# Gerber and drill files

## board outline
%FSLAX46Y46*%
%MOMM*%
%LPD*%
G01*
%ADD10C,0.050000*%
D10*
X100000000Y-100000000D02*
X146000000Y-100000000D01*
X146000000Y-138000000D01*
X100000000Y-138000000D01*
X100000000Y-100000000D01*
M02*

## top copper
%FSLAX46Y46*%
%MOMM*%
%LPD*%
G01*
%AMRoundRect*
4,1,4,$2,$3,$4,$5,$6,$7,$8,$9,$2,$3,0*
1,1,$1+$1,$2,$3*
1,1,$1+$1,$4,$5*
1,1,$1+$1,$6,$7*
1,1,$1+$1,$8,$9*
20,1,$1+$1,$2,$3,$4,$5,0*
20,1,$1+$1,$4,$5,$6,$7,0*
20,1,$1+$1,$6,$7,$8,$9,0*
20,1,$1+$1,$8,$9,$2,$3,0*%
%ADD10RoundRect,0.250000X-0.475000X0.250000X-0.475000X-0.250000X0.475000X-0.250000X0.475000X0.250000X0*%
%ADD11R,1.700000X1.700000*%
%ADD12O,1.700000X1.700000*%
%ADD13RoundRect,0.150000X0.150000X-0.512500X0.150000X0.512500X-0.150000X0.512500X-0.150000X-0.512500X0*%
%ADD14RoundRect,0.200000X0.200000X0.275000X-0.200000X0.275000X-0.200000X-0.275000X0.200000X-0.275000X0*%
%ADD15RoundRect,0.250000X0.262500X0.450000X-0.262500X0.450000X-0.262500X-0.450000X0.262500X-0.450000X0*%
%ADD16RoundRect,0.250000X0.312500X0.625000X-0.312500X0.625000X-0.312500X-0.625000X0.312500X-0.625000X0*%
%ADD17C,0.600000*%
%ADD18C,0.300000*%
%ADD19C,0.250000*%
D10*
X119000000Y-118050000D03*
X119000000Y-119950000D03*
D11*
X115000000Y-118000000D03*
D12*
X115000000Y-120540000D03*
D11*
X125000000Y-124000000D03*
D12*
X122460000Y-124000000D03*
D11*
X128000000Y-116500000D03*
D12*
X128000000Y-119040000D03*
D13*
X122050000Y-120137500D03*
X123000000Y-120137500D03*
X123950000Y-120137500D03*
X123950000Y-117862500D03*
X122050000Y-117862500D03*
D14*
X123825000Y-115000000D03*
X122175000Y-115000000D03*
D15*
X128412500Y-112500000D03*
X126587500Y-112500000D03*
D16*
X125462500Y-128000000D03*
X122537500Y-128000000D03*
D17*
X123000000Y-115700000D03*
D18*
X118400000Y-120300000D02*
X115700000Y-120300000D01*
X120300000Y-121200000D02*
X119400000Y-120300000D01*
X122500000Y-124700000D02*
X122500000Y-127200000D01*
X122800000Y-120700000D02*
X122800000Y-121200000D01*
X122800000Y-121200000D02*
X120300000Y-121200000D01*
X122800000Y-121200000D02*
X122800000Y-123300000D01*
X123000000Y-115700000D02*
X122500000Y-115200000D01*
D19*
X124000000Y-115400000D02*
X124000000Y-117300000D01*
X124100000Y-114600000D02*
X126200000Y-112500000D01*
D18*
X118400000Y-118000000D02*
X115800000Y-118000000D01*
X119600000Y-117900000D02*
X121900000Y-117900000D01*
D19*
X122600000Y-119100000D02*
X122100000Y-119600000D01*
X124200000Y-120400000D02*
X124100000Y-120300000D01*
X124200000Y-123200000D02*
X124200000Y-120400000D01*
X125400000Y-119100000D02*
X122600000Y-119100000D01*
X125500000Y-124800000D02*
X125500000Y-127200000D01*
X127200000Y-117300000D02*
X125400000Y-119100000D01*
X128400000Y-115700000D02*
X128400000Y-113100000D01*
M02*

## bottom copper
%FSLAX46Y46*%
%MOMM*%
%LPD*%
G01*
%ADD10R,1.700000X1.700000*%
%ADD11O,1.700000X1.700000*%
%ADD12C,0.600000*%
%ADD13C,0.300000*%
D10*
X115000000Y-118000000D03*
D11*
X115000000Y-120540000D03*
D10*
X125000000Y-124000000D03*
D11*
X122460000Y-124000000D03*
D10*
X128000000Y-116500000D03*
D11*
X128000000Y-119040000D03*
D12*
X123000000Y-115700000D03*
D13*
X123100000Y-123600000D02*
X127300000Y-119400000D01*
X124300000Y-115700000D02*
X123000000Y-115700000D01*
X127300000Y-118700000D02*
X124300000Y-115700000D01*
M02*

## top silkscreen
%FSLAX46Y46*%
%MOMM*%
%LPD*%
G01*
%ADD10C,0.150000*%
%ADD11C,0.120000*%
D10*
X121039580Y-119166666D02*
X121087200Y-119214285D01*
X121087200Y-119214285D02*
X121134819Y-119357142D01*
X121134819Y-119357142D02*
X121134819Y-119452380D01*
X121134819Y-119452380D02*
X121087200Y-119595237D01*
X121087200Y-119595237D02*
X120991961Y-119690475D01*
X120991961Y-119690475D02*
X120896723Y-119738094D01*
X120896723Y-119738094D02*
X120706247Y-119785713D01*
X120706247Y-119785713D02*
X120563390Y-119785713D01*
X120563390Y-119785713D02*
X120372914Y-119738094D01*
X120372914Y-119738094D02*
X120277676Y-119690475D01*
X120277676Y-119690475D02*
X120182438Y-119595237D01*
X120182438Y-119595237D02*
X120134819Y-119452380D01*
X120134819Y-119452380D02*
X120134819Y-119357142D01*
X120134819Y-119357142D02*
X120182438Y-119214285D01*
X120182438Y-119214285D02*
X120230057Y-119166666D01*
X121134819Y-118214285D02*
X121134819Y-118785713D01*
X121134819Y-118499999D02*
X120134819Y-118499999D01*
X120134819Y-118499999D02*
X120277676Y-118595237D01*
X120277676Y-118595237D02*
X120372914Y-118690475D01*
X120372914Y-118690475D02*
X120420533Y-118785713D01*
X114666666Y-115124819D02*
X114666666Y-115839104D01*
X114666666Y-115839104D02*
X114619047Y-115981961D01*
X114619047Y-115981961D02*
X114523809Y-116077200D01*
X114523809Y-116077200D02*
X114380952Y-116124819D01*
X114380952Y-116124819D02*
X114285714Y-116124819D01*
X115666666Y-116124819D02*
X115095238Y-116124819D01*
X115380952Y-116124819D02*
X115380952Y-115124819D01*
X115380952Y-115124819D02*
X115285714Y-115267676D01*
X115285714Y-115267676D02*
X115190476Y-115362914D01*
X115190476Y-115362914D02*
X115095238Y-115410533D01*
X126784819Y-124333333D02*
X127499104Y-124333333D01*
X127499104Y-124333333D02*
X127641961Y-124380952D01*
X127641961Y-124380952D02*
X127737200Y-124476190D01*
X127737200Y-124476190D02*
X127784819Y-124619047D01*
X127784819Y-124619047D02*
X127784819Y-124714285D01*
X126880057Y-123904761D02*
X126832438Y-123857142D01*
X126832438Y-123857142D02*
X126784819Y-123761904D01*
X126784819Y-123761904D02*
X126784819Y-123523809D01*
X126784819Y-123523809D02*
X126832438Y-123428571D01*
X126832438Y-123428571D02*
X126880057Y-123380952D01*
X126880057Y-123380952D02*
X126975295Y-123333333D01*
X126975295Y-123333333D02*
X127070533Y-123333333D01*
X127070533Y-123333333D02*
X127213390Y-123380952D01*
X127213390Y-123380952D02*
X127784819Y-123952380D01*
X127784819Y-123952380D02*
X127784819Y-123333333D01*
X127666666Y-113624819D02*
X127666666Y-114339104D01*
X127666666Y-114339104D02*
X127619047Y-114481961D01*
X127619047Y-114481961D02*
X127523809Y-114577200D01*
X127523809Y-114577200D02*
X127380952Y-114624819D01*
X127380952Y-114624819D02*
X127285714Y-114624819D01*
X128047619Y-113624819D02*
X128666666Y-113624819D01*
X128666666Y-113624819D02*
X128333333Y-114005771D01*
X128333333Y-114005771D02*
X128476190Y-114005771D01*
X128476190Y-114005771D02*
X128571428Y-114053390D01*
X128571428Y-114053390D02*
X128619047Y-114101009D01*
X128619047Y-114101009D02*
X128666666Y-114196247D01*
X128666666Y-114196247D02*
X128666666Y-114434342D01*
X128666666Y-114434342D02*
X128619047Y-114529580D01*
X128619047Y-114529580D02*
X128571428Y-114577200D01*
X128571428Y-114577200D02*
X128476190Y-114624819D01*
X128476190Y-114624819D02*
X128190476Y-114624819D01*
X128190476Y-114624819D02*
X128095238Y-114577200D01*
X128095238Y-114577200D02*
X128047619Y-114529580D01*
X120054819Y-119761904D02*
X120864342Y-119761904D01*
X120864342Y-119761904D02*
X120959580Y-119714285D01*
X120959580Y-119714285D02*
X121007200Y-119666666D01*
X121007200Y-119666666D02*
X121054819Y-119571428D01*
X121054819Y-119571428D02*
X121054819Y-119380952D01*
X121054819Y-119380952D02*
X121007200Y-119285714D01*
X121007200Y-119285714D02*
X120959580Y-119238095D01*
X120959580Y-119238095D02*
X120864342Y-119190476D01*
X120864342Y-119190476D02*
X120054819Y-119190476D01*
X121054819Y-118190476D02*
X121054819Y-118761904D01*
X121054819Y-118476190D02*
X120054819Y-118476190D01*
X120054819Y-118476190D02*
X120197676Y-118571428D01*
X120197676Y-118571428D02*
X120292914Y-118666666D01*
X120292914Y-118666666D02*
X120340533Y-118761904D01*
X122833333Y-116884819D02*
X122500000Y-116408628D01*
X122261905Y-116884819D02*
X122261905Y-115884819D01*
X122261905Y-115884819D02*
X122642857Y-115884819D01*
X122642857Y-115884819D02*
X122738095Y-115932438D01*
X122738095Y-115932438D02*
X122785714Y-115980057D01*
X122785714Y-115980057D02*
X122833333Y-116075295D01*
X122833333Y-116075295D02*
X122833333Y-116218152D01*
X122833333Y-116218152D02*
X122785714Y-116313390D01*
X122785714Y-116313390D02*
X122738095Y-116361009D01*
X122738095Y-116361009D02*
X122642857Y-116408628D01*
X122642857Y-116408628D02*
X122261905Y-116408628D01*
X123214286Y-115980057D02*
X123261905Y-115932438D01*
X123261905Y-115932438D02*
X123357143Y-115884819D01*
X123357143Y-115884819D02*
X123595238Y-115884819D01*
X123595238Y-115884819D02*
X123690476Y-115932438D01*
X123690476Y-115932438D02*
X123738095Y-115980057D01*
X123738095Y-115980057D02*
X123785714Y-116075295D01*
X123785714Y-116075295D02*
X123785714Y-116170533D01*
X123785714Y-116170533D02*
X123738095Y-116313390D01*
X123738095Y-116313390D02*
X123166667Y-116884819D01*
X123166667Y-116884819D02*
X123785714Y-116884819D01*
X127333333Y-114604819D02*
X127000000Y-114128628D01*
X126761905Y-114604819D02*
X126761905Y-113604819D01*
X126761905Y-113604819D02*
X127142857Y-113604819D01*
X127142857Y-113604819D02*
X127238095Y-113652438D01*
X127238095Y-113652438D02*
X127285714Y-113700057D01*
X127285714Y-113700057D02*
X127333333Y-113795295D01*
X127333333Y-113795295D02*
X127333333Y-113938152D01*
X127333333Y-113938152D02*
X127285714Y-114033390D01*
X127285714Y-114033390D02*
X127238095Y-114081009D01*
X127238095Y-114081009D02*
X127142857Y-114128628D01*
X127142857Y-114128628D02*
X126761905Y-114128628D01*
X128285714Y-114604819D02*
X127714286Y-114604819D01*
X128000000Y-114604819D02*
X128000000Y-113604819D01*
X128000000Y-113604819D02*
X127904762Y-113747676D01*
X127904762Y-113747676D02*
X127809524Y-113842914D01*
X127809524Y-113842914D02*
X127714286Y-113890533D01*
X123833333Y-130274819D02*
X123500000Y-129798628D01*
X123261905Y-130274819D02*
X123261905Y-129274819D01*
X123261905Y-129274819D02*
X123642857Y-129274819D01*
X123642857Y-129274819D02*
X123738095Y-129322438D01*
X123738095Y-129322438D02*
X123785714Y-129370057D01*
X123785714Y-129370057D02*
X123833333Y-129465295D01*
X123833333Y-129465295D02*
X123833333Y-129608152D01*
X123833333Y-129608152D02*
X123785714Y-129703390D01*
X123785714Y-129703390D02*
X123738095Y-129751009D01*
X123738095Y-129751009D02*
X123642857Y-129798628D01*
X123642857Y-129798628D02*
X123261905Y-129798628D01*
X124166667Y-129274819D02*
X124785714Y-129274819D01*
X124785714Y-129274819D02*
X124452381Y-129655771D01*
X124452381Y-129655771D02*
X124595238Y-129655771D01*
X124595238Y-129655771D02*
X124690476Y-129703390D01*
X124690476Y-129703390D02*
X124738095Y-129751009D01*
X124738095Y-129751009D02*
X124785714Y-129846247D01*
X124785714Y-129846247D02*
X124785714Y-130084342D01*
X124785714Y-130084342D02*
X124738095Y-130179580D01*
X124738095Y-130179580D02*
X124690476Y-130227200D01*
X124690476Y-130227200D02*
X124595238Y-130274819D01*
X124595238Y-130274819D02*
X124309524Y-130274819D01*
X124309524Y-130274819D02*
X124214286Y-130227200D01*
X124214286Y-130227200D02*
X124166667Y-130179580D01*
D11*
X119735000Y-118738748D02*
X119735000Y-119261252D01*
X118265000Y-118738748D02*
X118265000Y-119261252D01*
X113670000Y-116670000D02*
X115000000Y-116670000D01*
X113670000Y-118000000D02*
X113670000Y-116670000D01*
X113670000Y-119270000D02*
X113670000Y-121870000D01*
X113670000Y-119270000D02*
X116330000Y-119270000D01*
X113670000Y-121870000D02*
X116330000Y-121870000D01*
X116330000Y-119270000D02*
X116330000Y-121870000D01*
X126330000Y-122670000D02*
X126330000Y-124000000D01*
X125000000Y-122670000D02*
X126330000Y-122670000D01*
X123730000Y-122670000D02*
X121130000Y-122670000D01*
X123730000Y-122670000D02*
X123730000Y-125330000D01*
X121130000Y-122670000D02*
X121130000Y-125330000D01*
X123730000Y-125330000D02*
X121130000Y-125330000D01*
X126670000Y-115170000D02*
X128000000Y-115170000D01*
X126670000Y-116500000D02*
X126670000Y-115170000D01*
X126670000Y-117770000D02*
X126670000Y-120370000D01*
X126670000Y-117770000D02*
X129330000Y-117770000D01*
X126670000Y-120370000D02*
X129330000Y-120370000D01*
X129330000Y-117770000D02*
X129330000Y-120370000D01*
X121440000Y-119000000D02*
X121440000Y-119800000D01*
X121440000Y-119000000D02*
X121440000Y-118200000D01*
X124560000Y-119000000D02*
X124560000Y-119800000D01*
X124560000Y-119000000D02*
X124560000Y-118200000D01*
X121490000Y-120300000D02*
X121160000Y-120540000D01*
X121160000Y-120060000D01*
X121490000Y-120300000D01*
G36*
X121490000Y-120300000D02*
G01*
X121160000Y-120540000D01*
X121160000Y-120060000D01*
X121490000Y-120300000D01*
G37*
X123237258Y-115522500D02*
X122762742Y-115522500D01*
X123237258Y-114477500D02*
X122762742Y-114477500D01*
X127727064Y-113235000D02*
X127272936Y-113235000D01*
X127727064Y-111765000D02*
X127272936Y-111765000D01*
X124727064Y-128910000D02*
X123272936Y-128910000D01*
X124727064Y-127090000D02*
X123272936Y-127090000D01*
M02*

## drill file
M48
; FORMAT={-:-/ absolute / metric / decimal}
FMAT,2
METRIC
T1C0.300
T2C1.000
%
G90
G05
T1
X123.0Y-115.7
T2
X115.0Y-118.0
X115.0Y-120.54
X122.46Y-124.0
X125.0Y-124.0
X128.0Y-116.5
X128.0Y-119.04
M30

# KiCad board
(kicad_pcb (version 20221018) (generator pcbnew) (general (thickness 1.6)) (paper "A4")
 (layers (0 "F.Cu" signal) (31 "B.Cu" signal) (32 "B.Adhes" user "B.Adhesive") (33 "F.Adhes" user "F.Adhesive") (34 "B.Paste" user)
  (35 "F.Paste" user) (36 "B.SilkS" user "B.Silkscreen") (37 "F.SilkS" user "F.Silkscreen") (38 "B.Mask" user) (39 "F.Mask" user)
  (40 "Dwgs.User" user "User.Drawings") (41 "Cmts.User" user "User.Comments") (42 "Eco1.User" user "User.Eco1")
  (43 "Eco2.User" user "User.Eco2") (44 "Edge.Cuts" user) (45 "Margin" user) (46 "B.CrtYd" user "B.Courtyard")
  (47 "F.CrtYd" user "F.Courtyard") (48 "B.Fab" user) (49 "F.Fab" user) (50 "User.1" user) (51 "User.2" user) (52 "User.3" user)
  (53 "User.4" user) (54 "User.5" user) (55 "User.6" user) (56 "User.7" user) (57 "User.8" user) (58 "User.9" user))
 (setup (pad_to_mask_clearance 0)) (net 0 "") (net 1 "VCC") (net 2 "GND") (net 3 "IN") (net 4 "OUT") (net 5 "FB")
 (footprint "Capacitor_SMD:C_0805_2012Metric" (layer "F.Cu") (at 119 119 -90)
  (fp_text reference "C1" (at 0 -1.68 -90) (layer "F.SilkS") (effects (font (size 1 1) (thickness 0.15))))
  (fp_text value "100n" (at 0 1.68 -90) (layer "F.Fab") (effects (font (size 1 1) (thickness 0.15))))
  (fp_line (start -0.261252 -0.735) (end 0.261252 -0.735) (stroke (width 0.12) (type solid)) (layer "F.SilkS"))
  (fp_line (start -0.261252 0.735) (end 0.261252 0.735) (stroke (width 0.12) (type solid)) (layer "F.SilkS"))
  (pad "1" smd roundrect (at -0.95 0 270) (size 1 1.45) (layers "F.Cu" "F.Paste" "F.Mask") (roundrect_rratio 0.25) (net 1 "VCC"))
  (pad "2" smd roundrect (at 0.95 0 270) (size 1 1.45) (layers "F.Cu" "F.Paste" "F.Mask") (roundrect_rratio 0.25) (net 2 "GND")))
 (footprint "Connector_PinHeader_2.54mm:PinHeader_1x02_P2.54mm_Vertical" (layer "F.Cu") (at 115 118)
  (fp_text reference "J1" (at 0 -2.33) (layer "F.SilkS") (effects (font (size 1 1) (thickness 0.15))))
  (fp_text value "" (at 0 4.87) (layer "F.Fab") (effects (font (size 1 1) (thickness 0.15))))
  (fp_line (start -1.33 -1.33) (end 0 -1.33) (stroke (width 0.12) (type solid)) (layer "F.SilkS"))
  (fp_line (start -1.33 0) (end -1.33 -1.33) (stroke (width 0.12) (type solid)) (layer "F.SilkS"))
  (fp_line (start -1.33 1.27) (end -1.33 3.87) (stroke (width 0.12) (type solid)) (layer "F.SilkS"))
  (fp_line (start -1.33 1.27) (end 1.33 1.27) (stroke (width 0.12) (type solid)) (layer "F.SilkS"))
  (fp_line (start -1.33 3.87) (end 1.33 3.87) (stroke (width 0.12) (type solid)) (layer "F.SilkS"))
  (fp_line (start 1.33 1.27) (end 1.33 3.87) (stroke (width 0.12) (type solid)) (layer "F.SilkS"))
  (pad "1" thru_hole rect (at 0 0) (size 1.7 1.7) (drill 1) (layers "*.Cu" "*.Mask") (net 1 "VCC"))
  (pad "2" thru_hole oval (at 0 2.54) (size 1.7 1.7) (drill 1) (layers "*.Cu" "*.Mask") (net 2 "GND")))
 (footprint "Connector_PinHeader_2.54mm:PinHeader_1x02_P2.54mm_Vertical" (layer "F.Cu") (at 125 124 -90)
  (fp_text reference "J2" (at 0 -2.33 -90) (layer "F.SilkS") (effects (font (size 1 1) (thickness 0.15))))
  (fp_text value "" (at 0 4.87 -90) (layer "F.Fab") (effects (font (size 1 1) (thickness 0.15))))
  (fp_line (start -1.33 -1.33) (end 0 -1.33) (stroke (width 0.12) (type solid)) (layer "F.SilkS"))
  (fp_line (start -1.33 0) (end -1.33 -1.33) (stroke (width 0.12) (type solid)) (layer "F.SilkS"))
  (fp_line (start -1.33 1.27) (end -1.33 3.87) (stroke (width 0.12) (type solid)) (layer "F.SilkS"))
  (fp_line (start -1.33 1.27) (end 1.33 1.27) (stroke (width 0.12) (type solid)) (layer "F.SilkS"))
  (fp_line (start -1.33 3.87) (end 1.33 3.87) (stroke (width 0.12) (type solid)) (layer "F.SilkS"))
  (fp_line (start 1.33 1.27) (end 1.33 3.87) (stroke (width 0.12) (type solid)) (layer "F.SilkS"))
  (pad "1" thru_hole rect (at 0 0 270) (size 1.7 1.7) (drill 1) (layers "*.Cu" "*.Mask") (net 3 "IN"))
  (pad "2" thru_hole oval (at 0 2.54 270) (size 1.7 1.7) (drill 1) (layers "*.Cu" "*.Mask") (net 2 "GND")))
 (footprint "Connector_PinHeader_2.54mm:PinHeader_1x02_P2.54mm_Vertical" (layer "F.Cu") (at 128 116.5)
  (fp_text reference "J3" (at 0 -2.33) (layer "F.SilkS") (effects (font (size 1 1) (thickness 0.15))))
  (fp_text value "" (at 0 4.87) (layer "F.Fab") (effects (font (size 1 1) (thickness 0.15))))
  (fp_line (start -1.33 -1.33) (end 0 -1.33) (stroke (width 0.12) (type solid)) (layer "F.SilkS"))
  (fp_line (start -1.33 0) (end -1.33 -1.33) (stroke (width 0.12) (type solid)) (layer "F.SilkS"))
  (fp_line (start -1.33 1.27) (end -1.33 3.87) (stroke (width 0.12) (type solid)) (layer "F.SilkS"))
  (fp_line (start -1.33 1.27) (end 1.33 1.27) (stroke (width 0.12) (type solid)) (layer "F.SilkS"))
  (fp_line (start -1.33 3.87) (end 1.33 3.87) (stroke (width 0.12) (type solid)) (layer "F.SilkS"))
  (fp_line (start 1.33 1.27) (end 1.33 3.87) (stroke (width 0.12) (type solid)) (layer "F.SilkS"))
  (pad "1" thru_hole rect (at 0 0) (size 1.7 1.7) (drill 1) (layers "*.Cu" "*.Mask") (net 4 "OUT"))
  (pad "2" thru_hole oval (at 0 2.54) (size 1.7 1.7) (drill 1) (layers "*.Cu" "*.Mask") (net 2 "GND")))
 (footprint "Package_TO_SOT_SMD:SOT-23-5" (layer "F.Cu") (at 123 119 90)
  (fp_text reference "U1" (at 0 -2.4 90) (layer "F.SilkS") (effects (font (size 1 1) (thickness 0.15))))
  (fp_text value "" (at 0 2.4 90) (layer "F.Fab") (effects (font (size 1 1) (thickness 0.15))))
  (fp_line (start 0 -1.56) (end -0.8 -1.56) (stroke (width 0.12) (type solid)) (layer "F.SilkS"))
  (fp_line (start 0 -1.56) (end 0.8 -1.56) (stroke (width 0.12) (type solid)) (layer "F.SilkS"))
  (fp_line (start 0 1.56) (end -0.8 1.56) (stroke (width 0.12) (type solid)) (layer "F.SilkS"))
  (fp_line (start 0 1.56) (end 0.8 1.56) (stroke (width 0.12) (type solid)) (layer "F.SilkS"))
  (fp_poly
   (pts (xy -1.3 -1.51) (xy -1.54 -1.84) (xy -1.06 -1.84) (xy -1.3 -1.51)) (stroke (width 0.12) (type solid)) (fill solid) (layer "F.SilkS"))
  (pad "1" smd roundrect (at -1.1375 -0.95 90) (size 1.325 0.6) (layers "F.Cu" "F.Paste" "F.Mask") (roundrect_rratio 0.25) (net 4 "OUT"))
  (pad "2" smd roundrect (at -1.1375 0 90) (size 1.325 0.6) (layers "F.Cu" "F.Paste" "F.Mask") (roundrect_rratio 0.25) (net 2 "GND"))
  (pad "3" smd roundrect (at -1.1375 0.95 90) (size 1.325 0.6) (layers "F.Cu" "F.Paste" "F.Mask") (roundrect_rratio 0.25) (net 3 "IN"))
  (pad "4" smd roundrect (at 1.1375 0.95 90) (size 1.325 0.6) (layers "F.Cu" "F.Paste" "F.Mask") (roundrect_rratio 0.25) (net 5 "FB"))
  (pad "5" smd roundrect (at 1.1375 -0.95 90) (size 1.325 0.6) (layers "F.Cu" "F.Paste" "F.Mask") (roundrect_rratio 0.25) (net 1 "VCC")))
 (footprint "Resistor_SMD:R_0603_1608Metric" (layer "F.Cu") (at 123 115 180)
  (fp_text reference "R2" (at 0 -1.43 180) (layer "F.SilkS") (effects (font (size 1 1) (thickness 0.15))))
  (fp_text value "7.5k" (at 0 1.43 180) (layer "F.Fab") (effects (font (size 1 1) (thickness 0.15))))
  (fp_line (start -0.237258 -0.5225) (end 0.237258 -0.5225) (stroke (width 0.12) (type solid)) (layer "F.SilkS"))
  (fp_line (start -0.237258 0.5225) (end 0.237258 0.5225) (stroke (width 0.12) (type solid)) (layer "F.SilkS"))
  (pad "1" smd roundrect (at -0.825 0 180) (size 0.8 0.95) (layers "F.Cu" "F.Paste" "F.Mask") (roundrect_rratio 0.25) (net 5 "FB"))
  (pad "2" smd roundrect (at 0.825 0 180) (size 0.8 0.95) (layers "F.Cu" "F.Paste" "F.Mask") (roundrect_rratio 0.25) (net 2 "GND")))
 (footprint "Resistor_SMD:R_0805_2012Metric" (layer "F.Cu") (at 127.5 112.5 180)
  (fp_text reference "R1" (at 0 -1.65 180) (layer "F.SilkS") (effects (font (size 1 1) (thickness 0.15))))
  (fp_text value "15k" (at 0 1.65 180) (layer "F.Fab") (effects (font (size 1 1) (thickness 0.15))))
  (fp_line (start -0.227064 -0.735) (end 0.227064 -0.735) (stroke (width 0.12) (type solid)) (layer "F.SilkS"))
  (fp_line (start -0.227064 0.735) (end 0.227064 0.735) (stroke (width 0.12) (type solid)) (layer "F.SilkS"))
  (pad "1" smd roundrect (at -0.9125 0 180) (size 1.025 1.4) (layers "F.Cu" "F.Paste" "F.Mask") (roundrect_rratio 0.243902) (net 4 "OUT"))
  (pad "2" smd roundrect (at 0.9125 0 180) (size 1.025 1.4) (layers "F.Cu" "F.Paste" "F.Mask") (roundrect_rratio 0.243902) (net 5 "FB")))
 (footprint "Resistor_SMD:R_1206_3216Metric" (layer "F.Cu") (at 124 128 180)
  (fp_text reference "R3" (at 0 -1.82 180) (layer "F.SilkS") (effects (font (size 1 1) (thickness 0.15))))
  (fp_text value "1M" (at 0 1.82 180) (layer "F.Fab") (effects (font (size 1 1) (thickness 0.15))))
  (fp_line (start -0.727064 -0.91) (end 0.727064 -0.91) (stroke (width 0.12) (type solid)) (layer "F.SilkS"))
  (fp_line (start -0.727064 0.91) (end 0.727064 0.91) (stroke (width 0.12) (type solid)) (layer "F.SilkS"))
  (pad "1" smd roundrect (at -1.4625 0 180) (size 1.125 1.75) (layers "F.Cu" "F.Paste" "F.Mask") (roundrect_rratio 0.222222) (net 3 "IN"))
  (pad "2" smd roundrect (at 1.4625 0 180) (size 1.125 1.75) (layers "F.Cu" "F.Paste" "F.Mask") (roundrect_rratio 0.222222) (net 2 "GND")))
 (gr_rect (start 100 100) (end 146 138) (stroke (width 0.05) (type default)) (fill none) (layer "Edge.Cuts"))
 (segment (start 118.4 120.3) (end 115.7 120.3) (width 0.3) (layer "F.Cu") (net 2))
 (segment (start 120.3 121.2) (end 119.4 120.3) (width 0.3) (layer "F.Cu") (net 2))
 (segment (start 122.5 124.7) (end 122.5 127.2) (width 0.3) (layer "F.Cu") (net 2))
 (segment (start 122.8 120.7) (end 122.8 121.2) (width 0.3) (layer "F.Cu") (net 2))
 (segment (start 122.8 121.2) (end 120.3 121.2) (width 0.3) (layer "F.Cu") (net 2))
 (segment (start 122.8 121.2) (end 122.8 123.3) (width 0.3) (layer "F.Cu") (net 2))
 (segment (start 123 115.7) (end 122.5 115.2) (width 0.3) (layer "F.Cu") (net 2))
 (segment (start 124 115.4) (end 124 117.3) (width 0.25) (layer "F.Cu") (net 5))
 (segment (start 124.1 114.6) (end 126.2 112.5) (width 0.25) (layer "F.Cu") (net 5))
 (via (at 123 115.7) (size 0.6) (drill 0.3) (layers "F.Cu" "B.Cu") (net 2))
 (segment (start 118.4 118) (end 115.8 118) (width 0.3) (layer "F.Cu") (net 1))
 (segment (start 119.6 117.9) (end 121.9 117.9) (width 0.3) (layer "F.Cu") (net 1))
 (segment (start 122.6 119.1) (end 122.1 119.6) (width 0.25) (layer "F.Cu") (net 4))
 (segment (start 123.1 123.6) (end 127.3 119.4) (width 0.3) (layer "B.Cu") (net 2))
 (segment (start 124.2 120.4) (end 124.1 120.3) (width 0.25) (layer "F.Cu") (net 3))
 (segment (start 124.2 123.2) (end 124.2 120.4) (width 0.25) (layer "F.Cu") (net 3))
 (segment (start 124.3 115.7) (end 123 115.7) (width 0.3) (layer "B.Cu") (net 2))
 (segment (start 125.4 119.1) (end 122.6 119.1) (width 0.25) (layer "F.Cu") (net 4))
 (segment (start 125.5 124.8) (end 125.5 127.2) (width 0.25) (layer "F.Cu") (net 3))
 (segment (start 127.2 117.3) (end 125.4 119.1) (width 0.25) (layer "F.Cu") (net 4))
 (segment (start 127.3 118.7) (end 124.3 115.7) (width 0.3) (layer "B.Cu") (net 2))
 (segment (start 128.4 115.7) (end 128.4 113.1) (width 0.25) (layer "F.Cu") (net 4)))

